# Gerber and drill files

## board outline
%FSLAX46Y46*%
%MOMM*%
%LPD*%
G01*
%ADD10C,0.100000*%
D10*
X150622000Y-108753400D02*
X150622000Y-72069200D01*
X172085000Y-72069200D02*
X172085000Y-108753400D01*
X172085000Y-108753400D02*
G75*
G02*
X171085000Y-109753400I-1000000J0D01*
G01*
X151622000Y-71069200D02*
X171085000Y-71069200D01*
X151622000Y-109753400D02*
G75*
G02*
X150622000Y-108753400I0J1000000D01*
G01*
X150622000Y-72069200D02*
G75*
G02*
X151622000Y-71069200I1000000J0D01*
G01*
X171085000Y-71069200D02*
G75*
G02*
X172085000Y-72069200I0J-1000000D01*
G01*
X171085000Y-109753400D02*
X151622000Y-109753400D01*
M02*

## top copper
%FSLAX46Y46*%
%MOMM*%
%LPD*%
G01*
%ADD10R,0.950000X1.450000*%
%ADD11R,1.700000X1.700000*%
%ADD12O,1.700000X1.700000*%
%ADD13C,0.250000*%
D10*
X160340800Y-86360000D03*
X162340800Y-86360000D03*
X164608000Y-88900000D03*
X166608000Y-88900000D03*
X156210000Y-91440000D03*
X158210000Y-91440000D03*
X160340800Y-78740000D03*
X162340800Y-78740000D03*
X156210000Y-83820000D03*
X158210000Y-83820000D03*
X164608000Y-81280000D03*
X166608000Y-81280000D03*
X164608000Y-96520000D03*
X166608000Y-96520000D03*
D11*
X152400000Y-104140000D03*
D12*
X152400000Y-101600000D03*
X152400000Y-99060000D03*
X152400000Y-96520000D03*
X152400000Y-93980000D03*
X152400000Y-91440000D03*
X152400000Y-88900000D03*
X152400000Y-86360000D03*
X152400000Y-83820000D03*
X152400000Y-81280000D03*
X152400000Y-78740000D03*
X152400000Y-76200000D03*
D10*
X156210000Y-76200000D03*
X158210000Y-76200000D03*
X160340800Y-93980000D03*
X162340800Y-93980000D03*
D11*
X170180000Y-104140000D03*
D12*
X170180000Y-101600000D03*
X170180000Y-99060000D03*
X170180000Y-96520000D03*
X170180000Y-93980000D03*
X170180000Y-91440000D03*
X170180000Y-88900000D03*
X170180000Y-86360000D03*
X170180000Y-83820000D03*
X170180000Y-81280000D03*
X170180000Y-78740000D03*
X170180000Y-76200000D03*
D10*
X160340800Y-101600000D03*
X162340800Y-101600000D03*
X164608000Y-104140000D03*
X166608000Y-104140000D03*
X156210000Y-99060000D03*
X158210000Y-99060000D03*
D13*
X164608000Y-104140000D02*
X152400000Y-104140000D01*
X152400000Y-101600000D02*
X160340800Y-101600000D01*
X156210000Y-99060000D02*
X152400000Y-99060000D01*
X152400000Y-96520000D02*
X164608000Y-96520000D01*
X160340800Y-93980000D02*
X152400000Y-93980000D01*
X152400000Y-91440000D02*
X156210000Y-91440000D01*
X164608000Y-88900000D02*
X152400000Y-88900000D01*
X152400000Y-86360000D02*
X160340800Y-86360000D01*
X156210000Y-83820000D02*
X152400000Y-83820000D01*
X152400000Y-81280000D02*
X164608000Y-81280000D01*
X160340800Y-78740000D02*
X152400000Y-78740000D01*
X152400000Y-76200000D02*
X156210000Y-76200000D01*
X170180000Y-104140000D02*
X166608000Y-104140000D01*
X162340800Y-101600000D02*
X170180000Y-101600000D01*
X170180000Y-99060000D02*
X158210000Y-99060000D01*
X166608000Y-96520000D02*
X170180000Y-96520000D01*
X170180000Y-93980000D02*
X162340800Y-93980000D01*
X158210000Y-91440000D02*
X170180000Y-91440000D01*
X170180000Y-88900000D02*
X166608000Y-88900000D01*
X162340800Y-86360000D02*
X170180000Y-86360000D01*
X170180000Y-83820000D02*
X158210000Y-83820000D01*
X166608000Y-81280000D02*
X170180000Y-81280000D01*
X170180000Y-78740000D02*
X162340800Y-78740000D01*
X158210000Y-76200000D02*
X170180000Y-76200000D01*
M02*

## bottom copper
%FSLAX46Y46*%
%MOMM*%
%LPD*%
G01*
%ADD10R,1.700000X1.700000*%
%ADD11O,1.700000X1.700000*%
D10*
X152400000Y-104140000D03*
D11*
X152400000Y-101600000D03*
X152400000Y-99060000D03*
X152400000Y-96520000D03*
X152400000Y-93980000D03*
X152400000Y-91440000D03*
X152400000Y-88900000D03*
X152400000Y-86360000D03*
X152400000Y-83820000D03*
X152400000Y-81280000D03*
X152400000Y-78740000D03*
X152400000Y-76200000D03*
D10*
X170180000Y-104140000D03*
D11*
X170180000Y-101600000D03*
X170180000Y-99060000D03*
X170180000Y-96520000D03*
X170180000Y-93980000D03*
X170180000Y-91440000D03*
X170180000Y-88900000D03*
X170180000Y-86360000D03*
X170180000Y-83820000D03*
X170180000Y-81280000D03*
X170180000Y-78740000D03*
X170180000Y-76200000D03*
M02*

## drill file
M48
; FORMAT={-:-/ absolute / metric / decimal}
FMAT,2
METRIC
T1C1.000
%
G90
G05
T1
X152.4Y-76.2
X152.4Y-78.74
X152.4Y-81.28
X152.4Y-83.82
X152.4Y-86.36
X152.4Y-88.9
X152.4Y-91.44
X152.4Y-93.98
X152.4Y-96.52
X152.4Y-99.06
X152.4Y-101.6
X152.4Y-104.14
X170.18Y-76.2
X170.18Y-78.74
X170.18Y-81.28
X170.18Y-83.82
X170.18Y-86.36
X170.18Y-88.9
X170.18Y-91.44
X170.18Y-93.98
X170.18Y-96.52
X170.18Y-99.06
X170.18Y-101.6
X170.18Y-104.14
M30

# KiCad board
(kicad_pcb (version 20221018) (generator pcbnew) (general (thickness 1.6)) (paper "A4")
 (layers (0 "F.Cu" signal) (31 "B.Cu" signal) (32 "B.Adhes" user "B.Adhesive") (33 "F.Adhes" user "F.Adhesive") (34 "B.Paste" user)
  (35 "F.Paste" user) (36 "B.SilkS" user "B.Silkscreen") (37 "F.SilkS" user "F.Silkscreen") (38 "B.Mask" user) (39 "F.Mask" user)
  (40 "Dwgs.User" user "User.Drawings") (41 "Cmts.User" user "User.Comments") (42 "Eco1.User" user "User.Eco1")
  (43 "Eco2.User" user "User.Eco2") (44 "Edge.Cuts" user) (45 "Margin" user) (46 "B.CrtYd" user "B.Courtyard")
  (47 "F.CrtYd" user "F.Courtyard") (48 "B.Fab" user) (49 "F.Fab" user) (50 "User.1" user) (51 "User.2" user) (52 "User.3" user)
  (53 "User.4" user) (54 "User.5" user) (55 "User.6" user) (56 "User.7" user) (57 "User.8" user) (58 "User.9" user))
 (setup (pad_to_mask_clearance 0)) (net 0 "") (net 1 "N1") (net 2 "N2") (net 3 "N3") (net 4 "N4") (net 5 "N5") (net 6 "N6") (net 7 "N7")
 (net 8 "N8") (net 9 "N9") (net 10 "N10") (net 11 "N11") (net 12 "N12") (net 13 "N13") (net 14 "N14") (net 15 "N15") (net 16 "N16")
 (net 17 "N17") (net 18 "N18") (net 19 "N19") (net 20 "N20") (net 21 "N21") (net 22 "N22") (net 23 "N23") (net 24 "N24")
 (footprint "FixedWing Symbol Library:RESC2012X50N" (layer "F.Cu") (at 161.3408 86.36)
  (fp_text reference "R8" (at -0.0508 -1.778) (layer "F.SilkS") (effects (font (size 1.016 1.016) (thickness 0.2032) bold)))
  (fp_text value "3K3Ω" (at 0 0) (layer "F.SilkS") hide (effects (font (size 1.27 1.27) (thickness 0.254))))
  (pad "1" smd rect (at -1 0) (size 0.95 1.45) (layers "F.Cu" "F.Paste" "F.Mask") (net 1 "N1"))
  (pad "2" smd rect (at 1 0) (size 0.95 1.45) (layers "F.Cu" "F.Paste" "F.Mask") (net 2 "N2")))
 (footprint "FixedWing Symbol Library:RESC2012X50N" (layer "F.Cu") (at 165.608 88.9)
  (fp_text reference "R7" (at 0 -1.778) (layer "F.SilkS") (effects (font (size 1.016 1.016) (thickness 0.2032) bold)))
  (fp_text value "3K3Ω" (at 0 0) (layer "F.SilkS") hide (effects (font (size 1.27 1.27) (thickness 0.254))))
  (pad "1" smd rect (at -1 0) (size 0.95 1.45) (layers "F.Cu" "F.Paste" "F.Mask") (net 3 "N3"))
  (pad "2" smd rect (at 1 0) (size 0.95 1.45) (layers "F.Cu" "F.Paste" "F.Mask") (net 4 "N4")))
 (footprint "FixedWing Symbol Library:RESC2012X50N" (layer "F.Cu") (at 157.21 91.44)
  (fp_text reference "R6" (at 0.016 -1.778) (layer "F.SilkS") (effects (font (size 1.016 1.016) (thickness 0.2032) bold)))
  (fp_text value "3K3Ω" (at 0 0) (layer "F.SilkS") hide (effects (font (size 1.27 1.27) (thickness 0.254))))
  (pad "1" smd rect (at -1 0) (size 0.95 1.45) (layers "F.Cu" "F.Paste" "F.Mask") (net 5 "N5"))
  (pad "2" smd rect (at 1 0) (size 0.95 1.45) (layers "F.Cu" "F.Paste" "F.Mask") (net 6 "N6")))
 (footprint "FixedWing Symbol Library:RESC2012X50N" (layer "F.Cu") (at 161.3408 78.74)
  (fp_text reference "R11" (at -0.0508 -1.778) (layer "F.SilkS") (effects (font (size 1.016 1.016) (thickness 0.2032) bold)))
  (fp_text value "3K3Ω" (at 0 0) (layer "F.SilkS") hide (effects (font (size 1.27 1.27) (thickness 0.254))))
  (pad "1" smd rect (at -1 0) (size 0.95 1.45) (layers "F.Cu" "F.Paste" "F.Mask") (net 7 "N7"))
  (pad "2" smd rect (at 1 0) (size 0.95 1.45) (layers "F.Cu" "F.Paste" "F.Mask") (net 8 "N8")))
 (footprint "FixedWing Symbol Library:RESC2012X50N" (layer "F.Cu") (at 157.21 83.82)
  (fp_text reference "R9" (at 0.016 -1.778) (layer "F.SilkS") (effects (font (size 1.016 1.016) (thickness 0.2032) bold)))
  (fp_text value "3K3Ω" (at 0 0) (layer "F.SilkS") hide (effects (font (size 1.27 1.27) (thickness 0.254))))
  (pad "1" smd rect (at -1 0) (size 0.95 1.45) (layers "F.Cu" "F.Paste" "F.Mask") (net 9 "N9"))
  (pad "2" smd rect (at 1 0) (size 0.95 1.45) (layers "F.Cu" "F.Paste" "F.Mask") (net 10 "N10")))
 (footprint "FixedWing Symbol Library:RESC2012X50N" (layer "F.Cu") (at 165.608 81.28)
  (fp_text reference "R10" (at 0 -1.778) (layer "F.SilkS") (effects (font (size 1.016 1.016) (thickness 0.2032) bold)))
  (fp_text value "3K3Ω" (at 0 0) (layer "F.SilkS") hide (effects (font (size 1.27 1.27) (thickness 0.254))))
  (pad "1" smd rect (at -1 0) (size 0.95 1.45) (layers "F.Cu" "F.Paste" "F.Mask") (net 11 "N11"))
  (pad "2" smd rect (at 1 0) (size 0.95 1.45) (layers "F.Cu" "F.Paste" "F.Mask") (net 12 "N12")))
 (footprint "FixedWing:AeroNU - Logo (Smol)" (layer "F.Cu") (at 157.406049 109.377388)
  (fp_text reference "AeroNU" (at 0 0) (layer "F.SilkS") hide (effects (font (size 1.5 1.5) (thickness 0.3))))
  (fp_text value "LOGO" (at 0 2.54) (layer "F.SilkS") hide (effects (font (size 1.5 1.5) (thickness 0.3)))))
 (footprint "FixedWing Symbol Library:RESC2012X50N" (layer "F.Cu") (at 165.608 96.52)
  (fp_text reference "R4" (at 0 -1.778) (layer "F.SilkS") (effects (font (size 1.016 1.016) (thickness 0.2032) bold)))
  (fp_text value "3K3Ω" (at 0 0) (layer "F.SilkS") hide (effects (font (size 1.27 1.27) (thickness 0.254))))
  (pad "1" smd rect (at -1 0) (size 0.95 1.45) (layers "F.Cu" "F.Paste" "F.Mask") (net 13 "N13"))
  (pad "2" smd rect (at 1 0) (size 0.95 1.45) (layers "F.Cu" "F.Paste" "F.Mask") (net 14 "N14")))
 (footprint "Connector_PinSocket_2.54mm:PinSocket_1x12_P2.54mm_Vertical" (layer "F.Cu") (at 152.4 104.14 180)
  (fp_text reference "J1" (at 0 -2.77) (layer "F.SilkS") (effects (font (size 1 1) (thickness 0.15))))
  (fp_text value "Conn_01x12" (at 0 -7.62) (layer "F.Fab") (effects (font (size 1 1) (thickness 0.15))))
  (pad "1" thru_hole rect (at 0 0 180) (size 1.7 1.7) (drill 1) (layers "*.Cu" "*.Mask") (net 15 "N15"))
  (pad "2" thru_hole oval (at 0 2.54 180) (size 1.7 1.7) (drill 1) (layers "*.Cu" "*.Mask") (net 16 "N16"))
  (pad "3" thru_hole oval (at 0 5.08 180) (size 1.7 1.7) (drill 1) (layers "*.Cu" "*.Mask") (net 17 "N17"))
  (pad "4" thru_hole oval (at 0 7.62 180) (size 1.7 1.7) (drill 1) (layers "*.Cu" "*.Mask") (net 13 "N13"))
  (pad "5" thru_hole oval (at 0 10.16 180) (size 1.7 1.7) (drill 1) (layers "*.Cu" "*.Mask") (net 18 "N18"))
  (pad "6" thru_hole oval (at 0 12.7 180) (size 1.7 1.7) (drill 1) (layers "*.Cu" "*.Mask") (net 5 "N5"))
  (pad "7" thru_hole oval (at 0 15.24 180) (size 1.7 1.7) (drill 1) (layers "*.Cu" "*.Mask") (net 3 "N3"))
  (pad "8" thru_hole oval (at 0 17.78 180) (size 1.7 1.7) (drill 1) (layers "*.Cu" "*.Mask") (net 1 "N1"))
  (pad "9" thru_hole oval (at 0 20.32 180) (size 1.7 1.7) (drill 1) (layers "*.Cu" "*.Mask") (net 9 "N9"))
  (pad "10" thru_hole oval (at 0 22.86 180) (size 1.7 1.7) (drill 1) (layers "*.Cu" "*.Mask") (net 11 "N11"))
  (pad "11" thru_hole oval (at 0 25.4 180) (size 1.7 1.7) (drill 1) (layers "*.Cu" "*.Mask") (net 7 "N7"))
  (pad "12" thru_hole oval (at 0 27.94 180) (size 1.7 1.7) (drill 1) (layers "*.Cu" "*.Mask") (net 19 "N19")))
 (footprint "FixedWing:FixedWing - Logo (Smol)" (layer "F.Cu") (at 165.4175 73.1774)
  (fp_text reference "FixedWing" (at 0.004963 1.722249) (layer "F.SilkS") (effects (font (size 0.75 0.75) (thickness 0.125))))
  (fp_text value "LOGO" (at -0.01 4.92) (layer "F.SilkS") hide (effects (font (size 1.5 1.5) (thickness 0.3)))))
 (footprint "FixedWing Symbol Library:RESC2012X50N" (layer "F.Cu") (at 157.21 76.2)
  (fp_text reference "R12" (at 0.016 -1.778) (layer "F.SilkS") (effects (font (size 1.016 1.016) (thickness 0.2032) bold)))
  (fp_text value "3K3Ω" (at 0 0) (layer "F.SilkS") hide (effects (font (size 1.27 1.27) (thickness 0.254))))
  (pad "1" smd rect (at -1 0) (size 0.95 1.45) (layers "F.Cu" "F.Paste" "F.Mask") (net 19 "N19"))
  (pad "2" smd rect (at 1 0) (size 0.95 1.45) (layers "F.Cu" "F.Paste" "F.Mask") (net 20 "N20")))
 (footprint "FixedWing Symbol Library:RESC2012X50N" (layer "F.Cu") (at 161.3408 93.98)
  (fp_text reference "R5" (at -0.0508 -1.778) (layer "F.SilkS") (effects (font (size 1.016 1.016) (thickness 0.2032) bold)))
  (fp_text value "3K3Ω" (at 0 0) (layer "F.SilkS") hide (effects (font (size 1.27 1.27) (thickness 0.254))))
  (pad "1" smd rect (at -1 0) (size 0.95 1.45) (layers "F.Cu" "F.Paste" "F.Mask") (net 18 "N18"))
  (pad "2" smd rect (at 1 0) (size 0.95 1.45) (layers "F.Cu" "F.Paste" "F.Mask") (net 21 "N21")))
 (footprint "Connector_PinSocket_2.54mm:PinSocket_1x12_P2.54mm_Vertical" (layer "F.Cu") (at 170.18 104.14 180)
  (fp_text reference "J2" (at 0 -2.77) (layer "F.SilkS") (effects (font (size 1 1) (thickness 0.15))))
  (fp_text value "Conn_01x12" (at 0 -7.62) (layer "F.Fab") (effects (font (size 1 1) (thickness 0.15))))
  (pad "1" thru_hole rect (at 0 0 180) (size 1.7 1.7) (drill 1) (layers "*.Cu" "*.Mask") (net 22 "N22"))
  (pad "2" thru_hole oval (at 0 2.54 180) (size 1.7 1.7) (drill 1) (layers "*.Cu" "*.Mask") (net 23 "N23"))
  (pad "3" thru_hole oval (at 0 5.08 180) (size 1.7 1.7) (drill 1) (layers "*.Cu" "*.Mask") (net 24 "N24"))
  (pad "4" thru_hole oval (at 0 7.62 180) (size 1.7 1.7) (drill 1) (layers "*.Cu" "*.Mask") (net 14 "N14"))
  (pad "5" thru_hole oval (at 0 10.16 180) (size 1.7 1.7) (drill 1) (layers "*.Cu" "*.Mask") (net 21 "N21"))
  (pad "6" thru_hole oval (at 0 12.7 180) (size 1.7 1.7) (drill 1) (layers "*.Cu" "*.Mask") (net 6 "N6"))
  (pad "7" thru_hole oval (at 0 15.24 180) (size 1.7 1.7) (drill 1) (layers "*.Cu" "*.Mask") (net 4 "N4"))
  (pad "8" thru_hole oval (at 0 17.78 180) (size 1.7 1.7) (drill 1) (layers "*.Cu" "*.Mask") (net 2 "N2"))
  (pad "9" thru_hole oval (at 0 20.32 180) (size 1.7 1.7) (drill 1) (layers "*.Cu" "*.Mask") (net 10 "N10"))
  (pad "10" thru_hole oval (at 0 22.86 180) (size 1.7 1.7) (drill 1) (layers "*.Cu" "*.Mask") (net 12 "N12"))
  (pad "11" thru_hole oval (at 0 25.4 180) (size 1.7 1.7) (drill 1) (layers "*.Cu" "*.Mask") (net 8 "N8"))
  (pad "12" thru_hole oval (at 0 27.94 180) (size 1.7 1.7) (drill 1) (layers "*.Cu" "*.Mask") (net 20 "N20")))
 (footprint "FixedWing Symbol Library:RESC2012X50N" (layer "F.Cu") (at 161.3408 101.6)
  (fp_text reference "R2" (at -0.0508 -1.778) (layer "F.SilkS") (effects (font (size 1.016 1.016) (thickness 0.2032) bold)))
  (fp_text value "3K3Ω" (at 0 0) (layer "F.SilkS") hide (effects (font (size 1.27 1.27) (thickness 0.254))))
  (pad "1" smd rect (at -1 0) (size 0.95 1.45) (layers "F.Cu" "F.Paste" "F.Mask") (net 16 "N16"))
  (pad "2" smd rect (at 1 0) (size 0.95 1.45) (layers "F.Cu" "F.Paste" "F.Mask") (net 23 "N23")))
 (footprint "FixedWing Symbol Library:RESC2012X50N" (layer "F.Cu") (at 165.608 104.14)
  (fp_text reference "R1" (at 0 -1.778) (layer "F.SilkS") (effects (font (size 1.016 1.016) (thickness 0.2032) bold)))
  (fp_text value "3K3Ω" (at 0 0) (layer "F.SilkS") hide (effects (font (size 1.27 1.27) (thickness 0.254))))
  (pad "1" smd rect (at -1 0) (size 0.95 1.45) (layers "F.Cu" "F.Paste" "F.Mask") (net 15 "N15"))
  (pad "2" smd rect (at 1 0) (size 0.95 1.45) (layers "F.Cu" "F.Paste" "F.Mask") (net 22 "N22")))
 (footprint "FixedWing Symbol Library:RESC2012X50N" (layer "F.Cu") (at 157.21 99.06)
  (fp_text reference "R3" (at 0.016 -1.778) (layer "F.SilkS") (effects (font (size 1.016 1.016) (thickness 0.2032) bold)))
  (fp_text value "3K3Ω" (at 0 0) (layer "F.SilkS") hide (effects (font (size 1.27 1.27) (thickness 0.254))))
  (pad "1" smd rect (at -1 0) (size 0.95 1.45) (layers "F.Cu" "F.Paste" "F.Mask") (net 17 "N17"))
  (pad "2" smd rect (at 1 0) (size 0.95 1.45) (layers "F.Cu" "F.Paste" "F.Mask") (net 24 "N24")))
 (gr_line (start 150.622 108.7534) (end 150.622 72.0692) (stroke (width 0.1) (type default)) (layer "Edge.Cuts"))
 (gr_line (start 172.085 72.0692) (end 172.085 108.7534) (stroke (width 0.1) (type default)) (layer "Edge.Cuts"))
 (gr_arc (start 172.085 108.7534) (mid 171.792107 109.460507) (end 171.085 109.7534) (stroke (width 0.1) (type default)) (layer "Edge.Cuts"))
 (gr_line (start 151.622 71.0692) (end 171.085 71.0692) (stroke (width 0.1) (type default)) (layer "Edge.Cuts"))
 (gr_arc (start 151.622 109.7534) (mid 150.914893 109.460507) (end 150.622 108.7534) (stroke (width 0.1) (type default)) (layer "Edge.Cuts"))
 (gr_arc (start 150.622 72.0692) (mid 150.914893 71.362093) (end 151.622 71.0692) (stroke (width 0.1) (type default)) (layer "Edge.Cuts"))
 (gr_arc (start 171.085 71.0692) (mid 171.792107 71.362093) (end 172.085 72.0692) (stroke (width 0.1) (type default)) (layer "Edge.Cuts"))
 (gr_line (start 171.085 109.7534) (end 151.622 109.7534) (stroke (width 0.1) (type default)) (layer "Edge.Cuts"))
 (segment (start 164.608 104.14) (end 152.4 104.14) (width 0.25) (layer "F.Cu") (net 15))
 (segment (start 152.4 101.6) (end 160.3408 101.6) (width 0.25) (layer "F.Cu") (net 16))
 (segment (start 156.21 99.06) (end 152.4 99.06) (width 0.25) (layer "F.Cu") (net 17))
 (segment (start 152.4 96.52) (end 164.608 96.52) (width 0.25) (layer "F.Cu") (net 13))
 (segment (start 160.3408 93.98) (end 152.4 93.98) (width 0.25) (layer "F.Cu") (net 18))
 (segment (start 152.4 91.44) (end 156.21 91.44) (width 0.25) (layer "F.Cu") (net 5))
 (segment (start 164.608 88.9) (end 152.4 88.9) (width 0.25) (layer "F.Cu") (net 3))
 (segment (start 152.4 86.36) (end 160.3408 86.36) (width 0.25) (layer "F.Cu") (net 1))
 (segment (start 156.21 83.82) (end 152.4 83.82) (width 0.25) (layer "F.Cu") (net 9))
 (segment (start 152.4 81.28) (end 164.608 81.28) (width 0.25) (layer "F.Cu") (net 11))
 (segment (start 160.3408 78.74) (end 152.4 78.74) (width 0.25) (layer "F.Cu") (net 7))
 (segment (start 152.4 76.2) (end 156.21 76.2) (width 0.25) (layer "F.Cu") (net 19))
 (segment (start 170.18 104.14) (end 166.608 104.14) (width 0.25) (layer "F.Cu") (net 22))
 (segment (start 162.3408 101.6) (end 170.18 101.6) (width 0.25) (layer "F.Cu") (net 23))
 (segment (start 170.18 99.06) (end 158.21 99.06) (width 0.25) (layer "F.Cu") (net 24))
 (segment (start 166.608 96.52) (end 170.18 96.52) (width 0.25) (layer "F.Cu") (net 14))
 (segment (start 170.18 93.98) (end 162.3408 93.98) (width 0.25) (layer "F.Cu") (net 21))
 (segment (start 158.21 91.44) (end 170.18 91.44) (width 0.25) (layer "F.Cu") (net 6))
 (segment (start 170.18 88.9) (end 166.608 88.9) (width 0.25) (layer "F.Cu") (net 4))
 (segment (start 162.3408 86.36) (end 170.18 86.36) (width 0.25) (layer "F.Cu") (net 2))
 (segment (start 170.18 83.82) (end 158.21 83.82) (width 0.25) (layer "F.Cu") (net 10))
 (segment (start 166.608 81.28) (end 170.18 81.28) (width 0.25) (layer "F.Cu") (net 12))
 (segment (start 170.18 78.74) (end 162.3408 78.74) (width 0.25) (layer "F.Cu") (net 8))
 (segment (start 158.21 76.2) (end 170.18 76.2) (width 0.25) (layer "F.Cu") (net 20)))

